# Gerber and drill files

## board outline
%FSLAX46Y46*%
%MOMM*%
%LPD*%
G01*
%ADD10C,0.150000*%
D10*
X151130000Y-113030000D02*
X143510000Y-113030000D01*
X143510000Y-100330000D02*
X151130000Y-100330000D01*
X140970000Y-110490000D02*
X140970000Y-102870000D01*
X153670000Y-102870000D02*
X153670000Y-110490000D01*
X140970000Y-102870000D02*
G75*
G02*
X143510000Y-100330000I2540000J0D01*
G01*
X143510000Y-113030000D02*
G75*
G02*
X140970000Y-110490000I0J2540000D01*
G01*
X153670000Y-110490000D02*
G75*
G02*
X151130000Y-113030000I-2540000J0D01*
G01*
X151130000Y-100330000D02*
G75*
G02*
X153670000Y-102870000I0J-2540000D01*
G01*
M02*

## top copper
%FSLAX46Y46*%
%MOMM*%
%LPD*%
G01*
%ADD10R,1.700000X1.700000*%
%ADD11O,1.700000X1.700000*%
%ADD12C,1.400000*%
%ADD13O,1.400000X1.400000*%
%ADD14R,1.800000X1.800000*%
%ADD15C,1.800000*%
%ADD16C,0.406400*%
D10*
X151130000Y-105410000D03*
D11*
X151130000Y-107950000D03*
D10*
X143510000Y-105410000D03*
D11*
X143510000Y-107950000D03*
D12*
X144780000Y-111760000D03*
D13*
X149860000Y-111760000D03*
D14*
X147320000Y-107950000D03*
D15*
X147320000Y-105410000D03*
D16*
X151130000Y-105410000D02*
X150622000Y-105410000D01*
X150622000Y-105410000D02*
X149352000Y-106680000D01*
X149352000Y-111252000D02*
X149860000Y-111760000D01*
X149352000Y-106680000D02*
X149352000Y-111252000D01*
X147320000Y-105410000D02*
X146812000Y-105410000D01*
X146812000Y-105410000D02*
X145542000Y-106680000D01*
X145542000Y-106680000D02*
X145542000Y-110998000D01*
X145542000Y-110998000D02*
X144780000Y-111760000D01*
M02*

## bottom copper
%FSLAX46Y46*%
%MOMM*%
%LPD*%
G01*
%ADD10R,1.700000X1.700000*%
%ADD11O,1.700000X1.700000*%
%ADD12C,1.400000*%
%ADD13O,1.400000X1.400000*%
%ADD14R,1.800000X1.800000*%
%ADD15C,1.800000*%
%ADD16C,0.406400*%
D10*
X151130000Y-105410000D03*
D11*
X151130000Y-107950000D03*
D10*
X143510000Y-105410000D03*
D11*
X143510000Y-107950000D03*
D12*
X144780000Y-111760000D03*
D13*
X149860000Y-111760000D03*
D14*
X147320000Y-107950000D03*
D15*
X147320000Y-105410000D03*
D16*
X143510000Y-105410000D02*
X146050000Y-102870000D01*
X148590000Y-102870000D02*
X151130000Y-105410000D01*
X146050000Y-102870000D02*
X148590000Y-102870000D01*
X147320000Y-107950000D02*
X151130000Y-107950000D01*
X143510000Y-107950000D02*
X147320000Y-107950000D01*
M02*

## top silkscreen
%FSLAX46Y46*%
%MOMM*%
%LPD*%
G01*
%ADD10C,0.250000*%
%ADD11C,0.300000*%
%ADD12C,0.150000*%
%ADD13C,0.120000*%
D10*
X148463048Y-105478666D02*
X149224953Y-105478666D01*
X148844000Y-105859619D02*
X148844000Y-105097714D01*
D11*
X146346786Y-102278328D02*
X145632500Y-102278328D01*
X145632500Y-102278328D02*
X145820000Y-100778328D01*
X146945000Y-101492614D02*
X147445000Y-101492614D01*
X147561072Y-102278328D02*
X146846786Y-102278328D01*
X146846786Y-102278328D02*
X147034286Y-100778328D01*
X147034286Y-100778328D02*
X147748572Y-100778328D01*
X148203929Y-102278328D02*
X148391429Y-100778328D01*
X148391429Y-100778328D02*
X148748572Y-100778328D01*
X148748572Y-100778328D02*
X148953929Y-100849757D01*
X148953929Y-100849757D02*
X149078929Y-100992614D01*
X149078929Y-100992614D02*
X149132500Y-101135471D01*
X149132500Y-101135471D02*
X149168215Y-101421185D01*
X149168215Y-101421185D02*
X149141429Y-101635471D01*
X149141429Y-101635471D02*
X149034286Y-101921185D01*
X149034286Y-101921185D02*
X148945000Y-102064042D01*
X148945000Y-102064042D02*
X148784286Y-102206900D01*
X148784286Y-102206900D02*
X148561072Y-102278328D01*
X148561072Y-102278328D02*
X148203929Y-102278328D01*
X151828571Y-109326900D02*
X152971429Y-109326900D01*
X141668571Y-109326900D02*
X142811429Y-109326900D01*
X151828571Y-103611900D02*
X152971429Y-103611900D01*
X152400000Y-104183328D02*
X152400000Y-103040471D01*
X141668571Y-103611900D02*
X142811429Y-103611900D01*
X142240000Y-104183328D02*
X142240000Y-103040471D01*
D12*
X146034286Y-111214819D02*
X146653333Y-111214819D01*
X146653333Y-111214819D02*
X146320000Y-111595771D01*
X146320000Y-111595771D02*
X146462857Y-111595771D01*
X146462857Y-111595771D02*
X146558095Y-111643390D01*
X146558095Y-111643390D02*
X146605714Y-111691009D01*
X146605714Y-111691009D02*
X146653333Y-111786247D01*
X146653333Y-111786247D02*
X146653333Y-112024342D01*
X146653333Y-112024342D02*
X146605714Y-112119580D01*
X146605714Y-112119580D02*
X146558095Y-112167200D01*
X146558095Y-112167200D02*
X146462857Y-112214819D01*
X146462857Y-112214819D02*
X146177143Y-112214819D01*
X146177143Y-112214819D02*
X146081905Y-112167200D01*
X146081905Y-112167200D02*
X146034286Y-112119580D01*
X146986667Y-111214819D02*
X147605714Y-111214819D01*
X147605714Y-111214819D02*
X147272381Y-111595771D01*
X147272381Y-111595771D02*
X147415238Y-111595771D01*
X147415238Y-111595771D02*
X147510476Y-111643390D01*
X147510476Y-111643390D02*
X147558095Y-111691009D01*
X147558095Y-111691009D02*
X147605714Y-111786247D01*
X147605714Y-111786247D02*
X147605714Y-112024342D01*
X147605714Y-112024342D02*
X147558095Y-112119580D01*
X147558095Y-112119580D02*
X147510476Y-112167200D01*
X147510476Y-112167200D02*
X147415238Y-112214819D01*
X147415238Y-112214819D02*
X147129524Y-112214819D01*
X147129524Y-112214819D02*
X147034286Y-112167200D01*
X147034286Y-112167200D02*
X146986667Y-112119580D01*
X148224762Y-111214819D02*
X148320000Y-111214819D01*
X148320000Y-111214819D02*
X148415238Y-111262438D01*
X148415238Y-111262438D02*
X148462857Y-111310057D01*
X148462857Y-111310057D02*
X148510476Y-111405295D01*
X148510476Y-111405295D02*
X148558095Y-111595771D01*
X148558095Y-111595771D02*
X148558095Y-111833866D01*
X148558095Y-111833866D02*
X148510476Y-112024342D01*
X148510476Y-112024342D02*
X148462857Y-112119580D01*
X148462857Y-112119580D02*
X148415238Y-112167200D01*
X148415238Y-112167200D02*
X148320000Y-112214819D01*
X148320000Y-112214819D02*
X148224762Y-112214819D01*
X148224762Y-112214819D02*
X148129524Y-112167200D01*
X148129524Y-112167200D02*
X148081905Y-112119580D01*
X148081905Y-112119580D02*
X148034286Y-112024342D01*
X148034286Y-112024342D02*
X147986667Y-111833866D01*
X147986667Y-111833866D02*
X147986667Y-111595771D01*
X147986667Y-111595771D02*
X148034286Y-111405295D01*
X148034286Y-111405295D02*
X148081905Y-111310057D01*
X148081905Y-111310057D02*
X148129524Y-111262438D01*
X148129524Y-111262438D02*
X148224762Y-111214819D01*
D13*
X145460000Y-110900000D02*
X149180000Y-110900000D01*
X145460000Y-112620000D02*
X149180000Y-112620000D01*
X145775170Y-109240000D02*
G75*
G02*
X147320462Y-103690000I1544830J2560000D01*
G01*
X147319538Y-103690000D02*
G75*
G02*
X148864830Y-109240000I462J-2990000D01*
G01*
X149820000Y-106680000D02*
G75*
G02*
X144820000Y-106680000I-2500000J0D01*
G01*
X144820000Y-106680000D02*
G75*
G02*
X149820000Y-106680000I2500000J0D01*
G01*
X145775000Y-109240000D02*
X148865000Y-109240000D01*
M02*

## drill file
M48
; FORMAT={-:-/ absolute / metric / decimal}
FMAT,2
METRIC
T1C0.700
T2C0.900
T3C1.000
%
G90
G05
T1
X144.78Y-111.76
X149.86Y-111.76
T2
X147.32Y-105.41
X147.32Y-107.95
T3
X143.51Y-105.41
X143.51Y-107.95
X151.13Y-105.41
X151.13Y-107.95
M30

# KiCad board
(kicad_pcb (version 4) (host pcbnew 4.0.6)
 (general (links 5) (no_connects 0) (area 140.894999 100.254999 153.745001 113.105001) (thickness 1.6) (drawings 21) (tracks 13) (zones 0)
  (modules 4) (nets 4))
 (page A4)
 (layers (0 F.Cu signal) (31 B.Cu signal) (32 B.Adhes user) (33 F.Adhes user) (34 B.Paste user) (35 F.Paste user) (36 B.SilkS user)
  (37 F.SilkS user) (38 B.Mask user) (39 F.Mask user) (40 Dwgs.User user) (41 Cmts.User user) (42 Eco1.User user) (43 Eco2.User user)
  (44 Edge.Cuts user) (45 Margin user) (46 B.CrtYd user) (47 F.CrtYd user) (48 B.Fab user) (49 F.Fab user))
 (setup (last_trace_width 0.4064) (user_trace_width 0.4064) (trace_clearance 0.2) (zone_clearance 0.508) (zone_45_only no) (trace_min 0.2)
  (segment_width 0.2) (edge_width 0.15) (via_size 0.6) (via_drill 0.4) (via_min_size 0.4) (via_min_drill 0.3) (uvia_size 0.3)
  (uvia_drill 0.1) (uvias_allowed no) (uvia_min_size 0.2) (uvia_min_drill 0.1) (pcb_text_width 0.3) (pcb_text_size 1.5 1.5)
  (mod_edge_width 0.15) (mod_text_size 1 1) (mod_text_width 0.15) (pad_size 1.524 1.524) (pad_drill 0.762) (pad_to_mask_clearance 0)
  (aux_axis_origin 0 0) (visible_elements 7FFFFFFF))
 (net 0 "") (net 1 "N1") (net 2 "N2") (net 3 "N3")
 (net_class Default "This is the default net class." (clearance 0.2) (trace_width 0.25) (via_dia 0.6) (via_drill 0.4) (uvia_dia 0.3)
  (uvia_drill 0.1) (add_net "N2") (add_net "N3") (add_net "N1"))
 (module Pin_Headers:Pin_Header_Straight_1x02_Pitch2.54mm (layer F.Cu) (at 151.13 105.41)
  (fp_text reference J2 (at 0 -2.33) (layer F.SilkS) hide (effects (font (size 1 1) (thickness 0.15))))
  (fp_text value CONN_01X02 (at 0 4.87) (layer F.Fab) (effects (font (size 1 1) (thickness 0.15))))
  (pad 1 thru_hole rect (at 0 0) (size 1.7 1.7) (drill 1) (layers *.Cu *.Mask) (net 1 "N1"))
  (pad 2 thru_hole oval (at 0 2.54) (size 1.7 1.7) (drill 1) (layers *.Cu *.Mask) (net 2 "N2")))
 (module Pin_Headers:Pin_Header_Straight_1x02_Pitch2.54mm (layer F.Cu) (at 143.51 105.41)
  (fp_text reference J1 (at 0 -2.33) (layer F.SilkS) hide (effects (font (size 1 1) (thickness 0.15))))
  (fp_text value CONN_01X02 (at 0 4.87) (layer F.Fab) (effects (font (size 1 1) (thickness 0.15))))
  (pad 1 thru_hole rect (at 0 0) (size 1.7 1.7) (drill 1) (layers *.Cu *.Mask) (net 1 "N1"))
  (pad 2 thru_hole oval (at 0 2.54) (size 1.7 1.7) (drill 1) (layers *.Cu *.Mask) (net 2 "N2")))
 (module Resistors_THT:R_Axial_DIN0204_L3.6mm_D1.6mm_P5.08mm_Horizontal (layer F.Cu) (at 144.78 111.76)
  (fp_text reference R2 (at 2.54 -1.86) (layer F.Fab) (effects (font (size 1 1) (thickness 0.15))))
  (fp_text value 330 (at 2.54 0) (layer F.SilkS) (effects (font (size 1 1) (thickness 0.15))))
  (fp_line (start 0.68 -0.86) (end 4.4 -0.86) (layer F.SilkS) (width 0.12))
  (fp_line (start 0.68 0.86) (end 4.4 0.86) (layer F.SilkS) (width 0.12))
  (pad 1 thru_hole circle (at 0 0) (size 1.4 1.4) (drill 0.7) (layers *.Cu *.Mask) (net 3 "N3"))
  (pad 2 thru_hole oval (at 5.08 0) (size 1.4 1.4) (drill 0.7) (layers *.Cu *.Mask) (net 1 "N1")))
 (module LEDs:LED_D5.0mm (layer F.Cu) (at 147.32 107.95 90)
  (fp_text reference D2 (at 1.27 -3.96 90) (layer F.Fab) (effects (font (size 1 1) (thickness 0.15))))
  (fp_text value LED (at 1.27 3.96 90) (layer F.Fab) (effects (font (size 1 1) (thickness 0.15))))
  (fp_arc (start 1.27 0) (end -1.29 -1.54483) (angle 148.9) (layer F.SilkS) (width 0.12))
  (fp_arc (start 1.27 0) (end -1.29 1.54483) (angle -148.9) (layer F.SilkS) (width 0.12))
  (fp_circle (center 1.27 0) (end 3.77 0) (layer F.SilkS) (width 0.12))
  (fp_line (start -1.29 -1.545) (end -1.29 1.545) (layer F.SilkS) (width 0.12))
  (pad 1 thru_hole rect (at 0 0 90) (size 1.8 1.8) (drill 0.9) (layers *.Cu *.Mask) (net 2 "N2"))
  (pad 2 thru_hole circle (at 2.54 0 90) (size 1.8 1.8) (drill 0.9) (layers *.Cu *.Mask) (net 3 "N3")))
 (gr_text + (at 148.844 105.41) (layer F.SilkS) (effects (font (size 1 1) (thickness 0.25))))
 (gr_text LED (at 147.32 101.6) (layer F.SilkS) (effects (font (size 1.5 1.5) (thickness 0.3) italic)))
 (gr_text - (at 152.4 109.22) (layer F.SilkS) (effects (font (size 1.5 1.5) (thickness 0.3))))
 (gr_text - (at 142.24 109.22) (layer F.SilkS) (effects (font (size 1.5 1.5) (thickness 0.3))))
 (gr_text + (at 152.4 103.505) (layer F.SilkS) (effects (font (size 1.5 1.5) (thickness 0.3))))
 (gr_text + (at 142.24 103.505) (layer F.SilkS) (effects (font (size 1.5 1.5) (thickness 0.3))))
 (gr_line (start 151.13 113.03) (end 143.51 113.03) (angle 90) (layer Edge.Cuts) (width 0.15))
 (gr_line (start 143.51 100.33) (end 151.13 100.33) (angle 90) (layer Edge.Cuts) (width 0.15))
 (gr_line (start 140.97 110.49) (end 140.97 102.87) (angle 90) (layer Edge.Cuts) (width 0.15))
 (gr_line (start 153.67 102.87) (end 153.67 110.49) (angle 90) (layer Edge.Cuts) (width 0.15))
 (gr_arc (start 143.51 102.87) (end 140.97 102.87) (angle 90) (layer Edge.Cuts) (width 0.15))
 (gr_arc (start 143.51 110.49) (end 143.51 113.03) (angle 90) (layer Edge.Cuts) (width 0.15))
 (gr_arc (start 151.13 110.49) (end 153.67 110.49) (angle 90) (layer Edge.Cuts) (width 0.15))
 (gr_arc (start 151.13 102.87) (end 151.13 100.33) (angle 90) (layer Edge.Cuts) (width 0.15))
 (segment (start 151.13 105.41) (end 150.622 105.41) (width 0.4064) (layer F.Cu) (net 1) (status C00000))
 (segment (start 150.622 105.41) (end 149.352 106.68) (width 0.4064) (layer F.Cu) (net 1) (status 400000))
 (segment (start 149.352 111.252) (end 149.86 111.76) (width 0.4064) (layer F.Cu) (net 1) (status 800000))
 (segment (start 149.352 106.68) (end 149.352 111.252) (width 0.4064) (layer F.Cu) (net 1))
 (segment (start 143.51 105.41) (end 146.05 102.87) (width 0.4064) (layer B.Cu) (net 1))
 (segment (start 148.59 102.87) (end 151.13 105.41) (width 0.4064) (layer B.Cu) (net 1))
 (segment (start 146.05 102.87) (end 148.59 102.87) (width 0.4064) (layer B.Cu) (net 1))
 (segment (start 147.32 107.95) (end 151.13 107.95) (width 0.4064) (layer B.Cu) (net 2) (status C00000))
 (segment (start 143.51 107.95) (end 147.32 107.95) (width 0.4064) (layer B.Cu) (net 2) (status C00000))
 (segment (start 147.32 105.41) (end 146.812 105.41) (width 0.4064) (layer F.Cu) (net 3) (status C00000))
 (segment (start 146.812 105.41) (end 145.542 106.68) (width 0.4064) (layer F.Cu) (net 3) (status 400000))
 (segment (start 145.542 106.68) (end 145.542 110.998) (width 0.4064) (layer F.Cu) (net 3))
 (segment (start 145.542 110.998) (end 144.78 111.76) (width 0.4064) (layer F.Cu) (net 3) (status 800000)))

